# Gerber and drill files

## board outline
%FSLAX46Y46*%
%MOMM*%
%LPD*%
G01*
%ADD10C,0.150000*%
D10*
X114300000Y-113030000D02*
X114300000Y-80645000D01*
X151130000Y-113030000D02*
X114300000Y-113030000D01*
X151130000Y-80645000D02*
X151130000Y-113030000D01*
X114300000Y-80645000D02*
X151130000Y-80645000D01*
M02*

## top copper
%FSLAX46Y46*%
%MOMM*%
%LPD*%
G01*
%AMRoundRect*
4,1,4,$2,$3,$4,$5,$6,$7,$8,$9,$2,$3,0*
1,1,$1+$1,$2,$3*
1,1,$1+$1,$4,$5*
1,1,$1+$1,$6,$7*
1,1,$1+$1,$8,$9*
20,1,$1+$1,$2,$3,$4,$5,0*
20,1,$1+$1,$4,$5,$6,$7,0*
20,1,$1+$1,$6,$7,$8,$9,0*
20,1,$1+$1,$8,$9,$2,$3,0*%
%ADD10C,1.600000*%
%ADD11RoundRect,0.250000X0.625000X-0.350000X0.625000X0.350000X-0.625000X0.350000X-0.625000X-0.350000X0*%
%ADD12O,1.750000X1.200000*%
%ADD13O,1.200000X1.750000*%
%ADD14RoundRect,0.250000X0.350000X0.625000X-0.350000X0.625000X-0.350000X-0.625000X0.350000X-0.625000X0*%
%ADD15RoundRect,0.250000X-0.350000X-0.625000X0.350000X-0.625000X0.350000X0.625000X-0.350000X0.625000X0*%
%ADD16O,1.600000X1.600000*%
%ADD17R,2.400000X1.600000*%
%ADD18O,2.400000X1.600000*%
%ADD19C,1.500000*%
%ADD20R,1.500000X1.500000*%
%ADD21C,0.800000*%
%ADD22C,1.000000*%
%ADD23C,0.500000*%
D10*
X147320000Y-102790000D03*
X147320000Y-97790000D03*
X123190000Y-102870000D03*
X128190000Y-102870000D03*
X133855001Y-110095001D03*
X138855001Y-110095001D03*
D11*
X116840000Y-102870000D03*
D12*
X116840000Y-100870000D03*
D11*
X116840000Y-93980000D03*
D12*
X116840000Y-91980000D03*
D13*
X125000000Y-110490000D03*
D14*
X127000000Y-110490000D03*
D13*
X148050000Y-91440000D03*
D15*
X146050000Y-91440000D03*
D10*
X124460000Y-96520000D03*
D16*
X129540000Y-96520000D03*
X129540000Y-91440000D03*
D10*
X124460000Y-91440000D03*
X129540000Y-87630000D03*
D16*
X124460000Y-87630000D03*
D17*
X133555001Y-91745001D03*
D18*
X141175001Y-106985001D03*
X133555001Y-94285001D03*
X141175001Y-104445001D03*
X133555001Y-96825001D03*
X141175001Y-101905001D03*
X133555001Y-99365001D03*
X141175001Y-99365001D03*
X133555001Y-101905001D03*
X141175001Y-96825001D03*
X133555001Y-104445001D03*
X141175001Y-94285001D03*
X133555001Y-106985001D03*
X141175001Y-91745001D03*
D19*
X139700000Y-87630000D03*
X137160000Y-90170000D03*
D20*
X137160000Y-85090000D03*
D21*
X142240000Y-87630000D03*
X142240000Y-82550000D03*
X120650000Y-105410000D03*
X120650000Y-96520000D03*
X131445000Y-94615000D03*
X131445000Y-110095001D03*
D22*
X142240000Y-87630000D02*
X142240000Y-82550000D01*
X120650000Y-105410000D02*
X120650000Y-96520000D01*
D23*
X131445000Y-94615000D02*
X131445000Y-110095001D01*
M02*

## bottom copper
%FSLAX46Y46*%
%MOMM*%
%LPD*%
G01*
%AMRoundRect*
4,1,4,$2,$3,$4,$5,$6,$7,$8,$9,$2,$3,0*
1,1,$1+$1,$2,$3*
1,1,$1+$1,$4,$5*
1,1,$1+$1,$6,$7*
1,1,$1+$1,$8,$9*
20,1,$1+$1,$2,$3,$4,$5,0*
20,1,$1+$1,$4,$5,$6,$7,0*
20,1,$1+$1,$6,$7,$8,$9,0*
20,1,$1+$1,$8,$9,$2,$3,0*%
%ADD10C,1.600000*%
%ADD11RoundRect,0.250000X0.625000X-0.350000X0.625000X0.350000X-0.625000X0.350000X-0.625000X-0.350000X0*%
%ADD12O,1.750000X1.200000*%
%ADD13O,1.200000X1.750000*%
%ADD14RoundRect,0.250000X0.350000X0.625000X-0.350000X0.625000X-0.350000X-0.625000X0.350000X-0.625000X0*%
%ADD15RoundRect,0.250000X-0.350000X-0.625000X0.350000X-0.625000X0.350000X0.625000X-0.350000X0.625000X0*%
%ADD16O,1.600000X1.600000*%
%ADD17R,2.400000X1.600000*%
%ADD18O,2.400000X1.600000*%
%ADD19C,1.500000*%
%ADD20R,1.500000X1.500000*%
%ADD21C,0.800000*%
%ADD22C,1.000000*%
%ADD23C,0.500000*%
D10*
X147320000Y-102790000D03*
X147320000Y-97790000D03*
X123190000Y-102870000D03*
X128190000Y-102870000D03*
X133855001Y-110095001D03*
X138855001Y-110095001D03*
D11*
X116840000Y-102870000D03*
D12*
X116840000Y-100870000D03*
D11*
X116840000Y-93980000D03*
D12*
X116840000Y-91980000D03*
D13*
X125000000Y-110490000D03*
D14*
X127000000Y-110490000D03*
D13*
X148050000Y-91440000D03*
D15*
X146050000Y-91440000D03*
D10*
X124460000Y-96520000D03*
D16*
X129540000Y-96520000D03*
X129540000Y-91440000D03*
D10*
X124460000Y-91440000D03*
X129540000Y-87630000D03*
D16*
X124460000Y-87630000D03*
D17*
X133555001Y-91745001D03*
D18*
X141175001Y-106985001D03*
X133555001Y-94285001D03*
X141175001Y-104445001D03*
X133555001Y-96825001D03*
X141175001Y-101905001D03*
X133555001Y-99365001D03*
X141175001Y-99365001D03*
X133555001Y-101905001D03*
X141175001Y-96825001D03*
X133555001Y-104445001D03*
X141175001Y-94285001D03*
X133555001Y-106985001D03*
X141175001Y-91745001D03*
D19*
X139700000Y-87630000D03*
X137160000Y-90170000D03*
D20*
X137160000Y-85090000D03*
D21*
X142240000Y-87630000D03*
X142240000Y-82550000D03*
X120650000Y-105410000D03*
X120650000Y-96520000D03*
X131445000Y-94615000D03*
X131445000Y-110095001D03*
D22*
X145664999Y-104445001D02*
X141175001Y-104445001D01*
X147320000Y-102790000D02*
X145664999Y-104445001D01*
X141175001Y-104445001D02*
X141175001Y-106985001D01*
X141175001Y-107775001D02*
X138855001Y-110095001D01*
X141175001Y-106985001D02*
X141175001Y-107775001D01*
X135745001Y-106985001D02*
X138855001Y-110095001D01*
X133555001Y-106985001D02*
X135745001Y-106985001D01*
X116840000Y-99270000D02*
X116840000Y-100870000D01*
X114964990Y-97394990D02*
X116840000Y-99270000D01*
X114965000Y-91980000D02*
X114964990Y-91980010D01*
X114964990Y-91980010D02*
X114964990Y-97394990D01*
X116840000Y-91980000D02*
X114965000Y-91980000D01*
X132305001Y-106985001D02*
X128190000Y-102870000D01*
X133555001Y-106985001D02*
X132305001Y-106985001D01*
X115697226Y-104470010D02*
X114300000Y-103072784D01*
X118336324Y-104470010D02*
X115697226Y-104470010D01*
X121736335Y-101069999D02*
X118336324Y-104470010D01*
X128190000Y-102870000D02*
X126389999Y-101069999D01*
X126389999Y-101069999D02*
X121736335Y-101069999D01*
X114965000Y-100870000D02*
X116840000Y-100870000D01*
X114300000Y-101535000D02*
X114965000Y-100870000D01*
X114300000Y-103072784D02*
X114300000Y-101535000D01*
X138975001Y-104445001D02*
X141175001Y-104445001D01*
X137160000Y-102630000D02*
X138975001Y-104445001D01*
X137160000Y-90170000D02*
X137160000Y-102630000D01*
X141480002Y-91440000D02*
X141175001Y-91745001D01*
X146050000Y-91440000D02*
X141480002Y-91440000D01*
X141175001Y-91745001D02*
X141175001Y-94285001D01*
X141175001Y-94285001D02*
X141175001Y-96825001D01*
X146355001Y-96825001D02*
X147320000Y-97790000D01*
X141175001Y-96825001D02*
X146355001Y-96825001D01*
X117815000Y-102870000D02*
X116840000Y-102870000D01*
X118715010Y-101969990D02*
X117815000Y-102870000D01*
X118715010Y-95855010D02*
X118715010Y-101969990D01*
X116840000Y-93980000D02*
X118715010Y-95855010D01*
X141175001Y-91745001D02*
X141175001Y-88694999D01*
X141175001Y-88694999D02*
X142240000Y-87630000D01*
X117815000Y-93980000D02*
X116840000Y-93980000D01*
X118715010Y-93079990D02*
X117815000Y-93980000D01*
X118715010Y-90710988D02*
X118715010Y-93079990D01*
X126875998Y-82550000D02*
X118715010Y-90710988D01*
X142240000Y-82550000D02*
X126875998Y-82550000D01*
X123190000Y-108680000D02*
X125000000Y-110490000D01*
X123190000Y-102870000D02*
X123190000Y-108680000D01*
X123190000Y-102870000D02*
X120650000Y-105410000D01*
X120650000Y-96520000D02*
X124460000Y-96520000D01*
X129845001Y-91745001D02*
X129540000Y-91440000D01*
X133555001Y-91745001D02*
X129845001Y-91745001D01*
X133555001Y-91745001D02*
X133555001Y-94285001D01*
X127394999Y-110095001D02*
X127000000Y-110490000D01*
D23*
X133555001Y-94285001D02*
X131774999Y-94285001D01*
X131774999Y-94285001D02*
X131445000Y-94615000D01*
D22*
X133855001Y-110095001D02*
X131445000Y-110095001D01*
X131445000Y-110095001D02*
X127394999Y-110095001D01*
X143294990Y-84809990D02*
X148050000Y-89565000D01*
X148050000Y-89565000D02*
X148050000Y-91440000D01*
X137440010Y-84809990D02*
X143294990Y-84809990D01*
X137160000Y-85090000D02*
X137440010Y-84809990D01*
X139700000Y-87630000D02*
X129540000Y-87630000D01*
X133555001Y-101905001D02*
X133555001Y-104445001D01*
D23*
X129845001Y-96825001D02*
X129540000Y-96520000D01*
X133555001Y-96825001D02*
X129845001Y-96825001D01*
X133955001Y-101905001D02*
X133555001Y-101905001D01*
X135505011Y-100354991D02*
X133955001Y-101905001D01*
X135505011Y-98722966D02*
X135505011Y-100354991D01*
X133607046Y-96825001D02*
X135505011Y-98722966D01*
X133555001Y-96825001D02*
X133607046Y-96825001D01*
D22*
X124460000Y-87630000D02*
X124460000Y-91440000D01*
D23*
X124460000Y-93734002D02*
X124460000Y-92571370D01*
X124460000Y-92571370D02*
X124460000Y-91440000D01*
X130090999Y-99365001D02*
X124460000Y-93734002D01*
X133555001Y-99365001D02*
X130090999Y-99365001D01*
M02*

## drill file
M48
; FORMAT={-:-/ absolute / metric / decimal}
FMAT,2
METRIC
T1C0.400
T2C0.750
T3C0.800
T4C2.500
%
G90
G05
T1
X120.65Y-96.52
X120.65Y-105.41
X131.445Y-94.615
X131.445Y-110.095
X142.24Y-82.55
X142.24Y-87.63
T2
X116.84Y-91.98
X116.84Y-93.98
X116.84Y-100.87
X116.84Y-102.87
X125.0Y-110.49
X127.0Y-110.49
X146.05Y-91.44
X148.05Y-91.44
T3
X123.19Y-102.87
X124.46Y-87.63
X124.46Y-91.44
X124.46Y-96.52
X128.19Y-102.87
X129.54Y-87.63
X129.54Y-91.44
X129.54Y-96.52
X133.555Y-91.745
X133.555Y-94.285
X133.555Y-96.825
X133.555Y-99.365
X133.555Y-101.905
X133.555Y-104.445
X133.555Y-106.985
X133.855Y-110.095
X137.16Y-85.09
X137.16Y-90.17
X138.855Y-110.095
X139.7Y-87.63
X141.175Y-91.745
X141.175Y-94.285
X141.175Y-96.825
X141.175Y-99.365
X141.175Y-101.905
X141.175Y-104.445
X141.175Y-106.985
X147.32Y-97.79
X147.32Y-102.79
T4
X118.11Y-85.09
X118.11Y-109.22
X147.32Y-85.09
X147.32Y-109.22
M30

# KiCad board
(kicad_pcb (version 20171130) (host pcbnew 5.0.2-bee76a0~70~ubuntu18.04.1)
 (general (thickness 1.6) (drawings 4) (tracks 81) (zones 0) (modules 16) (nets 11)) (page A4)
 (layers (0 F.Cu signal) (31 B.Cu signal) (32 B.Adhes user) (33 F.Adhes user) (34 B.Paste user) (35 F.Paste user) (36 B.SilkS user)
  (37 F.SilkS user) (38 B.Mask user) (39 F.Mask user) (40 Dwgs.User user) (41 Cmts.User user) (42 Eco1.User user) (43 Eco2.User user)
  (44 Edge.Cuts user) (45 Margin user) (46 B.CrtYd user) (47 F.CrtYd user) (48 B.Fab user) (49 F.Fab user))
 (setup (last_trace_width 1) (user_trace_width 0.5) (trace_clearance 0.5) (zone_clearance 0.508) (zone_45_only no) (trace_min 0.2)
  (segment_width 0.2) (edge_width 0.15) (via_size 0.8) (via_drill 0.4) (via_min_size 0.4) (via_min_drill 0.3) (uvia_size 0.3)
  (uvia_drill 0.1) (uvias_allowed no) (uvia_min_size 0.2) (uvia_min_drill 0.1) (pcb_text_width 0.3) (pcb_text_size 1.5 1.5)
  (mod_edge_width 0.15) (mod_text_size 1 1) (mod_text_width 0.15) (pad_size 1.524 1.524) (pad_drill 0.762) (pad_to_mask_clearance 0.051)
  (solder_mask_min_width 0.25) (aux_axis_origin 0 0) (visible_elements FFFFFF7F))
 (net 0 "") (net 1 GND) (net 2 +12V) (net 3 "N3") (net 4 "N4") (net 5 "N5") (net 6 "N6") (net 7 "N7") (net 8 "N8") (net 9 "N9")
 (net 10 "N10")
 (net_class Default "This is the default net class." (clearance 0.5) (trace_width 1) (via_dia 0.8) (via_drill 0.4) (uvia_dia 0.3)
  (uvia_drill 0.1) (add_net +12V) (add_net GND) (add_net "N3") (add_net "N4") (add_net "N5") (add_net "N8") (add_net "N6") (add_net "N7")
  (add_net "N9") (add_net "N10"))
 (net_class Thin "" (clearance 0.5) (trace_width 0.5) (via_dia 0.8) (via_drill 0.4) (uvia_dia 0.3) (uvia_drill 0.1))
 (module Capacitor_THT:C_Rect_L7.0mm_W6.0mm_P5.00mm (layer F.Cu) (at 147.32 97.79 270)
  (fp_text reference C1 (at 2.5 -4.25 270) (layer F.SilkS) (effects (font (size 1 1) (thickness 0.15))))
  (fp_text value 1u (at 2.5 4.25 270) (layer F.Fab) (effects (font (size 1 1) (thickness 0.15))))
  (pad 2 thru_hole circle (at 5 0 270) (size 1.6 1.6) (drill 0.8) (layers *.Cu *.Mask) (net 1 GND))
  (pad 1 thru_hole circle (at 0 0 270) (size 1.6 1.6) (drill 0.8) (layers *.Cu *.Mask) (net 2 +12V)))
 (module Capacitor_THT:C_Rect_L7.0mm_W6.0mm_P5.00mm (layer F.Cu) (at 123.19 102.87)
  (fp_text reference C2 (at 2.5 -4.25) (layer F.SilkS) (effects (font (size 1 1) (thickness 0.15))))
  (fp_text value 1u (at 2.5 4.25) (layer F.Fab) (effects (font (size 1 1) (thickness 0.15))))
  (pad 1 thru_hole circle (at 0 0) (size 1.6 1.6) (drill 0.8) (layers *.Cu *.Mask) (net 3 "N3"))
  (pad 2 thru_hole circle (at 5 0) (size 1.6 1.6) (drill 0.8) (layers *.Cu *.Mask) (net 1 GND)))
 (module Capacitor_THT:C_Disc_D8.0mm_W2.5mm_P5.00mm (layer F.Cu) (at 133.855001 110.095001)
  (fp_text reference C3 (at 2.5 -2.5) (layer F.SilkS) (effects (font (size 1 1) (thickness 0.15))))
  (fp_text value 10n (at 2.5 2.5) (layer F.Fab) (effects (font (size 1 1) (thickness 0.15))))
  (pad 1 thru_hole circle (at 0 0) (size 1.6 1.6) (drill 0.8) (layers *.Cu *.Mask) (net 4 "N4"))
  (pad 2 thru_hole circle (at 5 0) (size 1.6 1.6) (drill 0.8) (layers *.Cu *.Mask) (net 1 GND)))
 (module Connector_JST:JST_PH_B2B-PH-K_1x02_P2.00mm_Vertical (layer F.Cu) (at 116.84 102.87 90)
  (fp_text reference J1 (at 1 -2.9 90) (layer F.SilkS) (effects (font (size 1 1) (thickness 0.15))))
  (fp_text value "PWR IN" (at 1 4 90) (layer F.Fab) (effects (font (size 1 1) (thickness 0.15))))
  (pad 1 thru_hole roundrect (at 0 0 90) (size 1.2 1.75) (drill 0.75) (layers *.Cu *.Mask) (roundrect_rratio 0.208333) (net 2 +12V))
  (pad 2 thru_hole oval (at 2 0 90) (size 1.2 1.75) (drill 0.75) (layers *.Cu *.Mask) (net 1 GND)))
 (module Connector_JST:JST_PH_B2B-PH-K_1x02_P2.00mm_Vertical (layer F.Cu) (at 116.84 93.98 90)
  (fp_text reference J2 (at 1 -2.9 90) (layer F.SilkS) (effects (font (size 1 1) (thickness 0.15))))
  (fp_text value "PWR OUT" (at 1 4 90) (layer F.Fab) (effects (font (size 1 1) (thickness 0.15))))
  (pad 1 thru_hole roundrect (at 0 0 90) (size 1.2 1.75) (drill 0.75) (layers *.Cu *.Mask) (roundrect_rratio 0.208333) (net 2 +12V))
  (pad 2 thru_hole oval (at 2 0 90) (size 1.2 1.75) (drill 0.75) (layers *.Cu *.Mask) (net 1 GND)))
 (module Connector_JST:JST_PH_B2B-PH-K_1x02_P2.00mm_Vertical (layer F.Cu) (at 127 110.49 180)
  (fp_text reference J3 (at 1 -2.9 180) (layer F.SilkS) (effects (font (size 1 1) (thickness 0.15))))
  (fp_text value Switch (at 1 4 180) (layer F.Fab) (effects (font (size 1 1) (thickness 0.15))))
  (pad 2 thru_hole oval (at 2 0 180) (size 1.2 1.75) (drill 0.75) (layers *.Cu *.Mask) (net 3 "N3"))
  (pad 1 thru_hole roundrect (at 0 0 180) (size 1.2 1.75) (drill 0.75) (layers *.Cu *.Mask) (roundrect_rratio 0.208333) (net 4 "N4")))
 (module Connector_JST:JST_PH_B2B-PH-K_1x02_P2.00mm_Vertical (layer F.Cu) (at 146.05 91.44)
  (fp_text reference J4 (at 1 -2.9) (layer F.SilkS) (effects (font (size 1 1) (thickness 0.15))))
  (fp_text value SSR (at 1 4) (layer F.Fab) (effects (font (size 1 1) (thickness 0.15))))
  (pad 2 thru_hole oval (at 2 0) (size 1.2 1.75) (drill 0.75) (layers *.Cu *.Mask) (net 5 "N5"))
  (pad 1 thru_hole roundrect (at 0 0) (size 1.2 1.75) (drill 0.75) (layers *.Cu *.Mask) (roundrect_rratio 0.208333) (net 2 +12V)))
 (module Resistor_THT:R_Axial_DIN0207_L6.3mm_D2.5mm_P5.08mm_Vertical (layer F.Cu) (at 124.46 96.52)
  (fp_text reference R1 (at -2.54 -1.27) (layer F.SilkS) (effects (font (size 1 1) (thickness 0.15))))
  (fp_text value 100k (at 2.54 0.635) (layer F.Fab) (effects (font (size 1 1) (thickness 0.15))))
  (pad 1 thru_hole circle (at 0 0) (size 1.6 1.6) (drill 0.8) (layers *.Cu *.Mask) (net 3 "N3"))
  (pad 2 thru_hole oval (at 5.08 0) (size 1.6 1.6) (drill 0.8) (layers *.Cu *.Mask) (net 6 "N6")))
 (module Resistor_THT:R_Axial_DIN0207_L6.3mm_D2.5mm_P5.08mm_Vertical (layer F.Cu) (at 124.46 91.44)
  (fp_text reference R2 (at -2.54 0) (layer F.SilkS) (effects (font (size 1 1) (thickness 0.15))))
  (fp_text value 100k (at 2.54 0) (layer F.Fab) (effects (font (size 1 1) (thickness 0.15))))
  (pad 2 thru_hole oval (at 5.08 0) (size 1.6 1.6) (drill 0.8) (layers *.Cu *.Mask) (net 4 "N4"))
  (pad 1 thru_hole circle (at 0 0) (size 1.6 1.6) (drill 0.8) (layers *.Cu *.Mask) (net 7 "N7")))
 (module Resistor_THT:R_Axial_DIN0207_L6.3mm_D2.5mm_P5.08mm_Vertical (layer F.Cu) (at 129.54 87.63 180)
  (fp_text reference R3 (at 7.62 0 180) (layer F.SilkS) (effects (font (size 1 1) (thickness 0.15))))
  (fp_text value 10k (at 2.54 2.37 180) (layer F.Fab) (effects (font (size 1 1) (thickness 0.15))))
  (pad 1 thru_hole circle (at 0 0 180) (size 1.6 1.6) (drill 0.8) (layers *.Cu *.Mask) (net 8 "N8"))
  (pad 2 thru_hole oval (at 5.08 0 180) (size 1.6 1.6) (drill 0.8) (layers *.Cu *.Mask) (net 7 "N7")))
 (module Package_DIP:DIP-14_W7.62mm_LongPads (layer F.Cu) (at 133.555001 91.745001)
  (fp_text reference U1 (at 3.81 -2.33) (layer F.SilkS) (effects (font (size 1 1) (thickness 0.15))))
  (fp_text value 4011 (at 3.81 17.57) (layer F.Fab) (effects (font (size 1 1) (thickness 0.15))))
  (pad 1 thru_hole rect (at 0 0) (size 2.4 1.6) (drill 0.8) (layers *.Cu *.Mask) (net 4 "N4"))
  (pad 8 thru_hole oval (at 7.62 15.24) (size 2.4 1.6) (drill 0.8) (layers *.Cu *.Mask) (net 1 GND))
  (pad 2 thru_hole oval (at 0 2.54) (size 2.4 1.6) (drill 0.8) (layers *.Cu *.Mask) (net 4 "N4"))
  (pad 9 thru_hole oval (at 7.62 12.7) (size 2.4 1.6) (drill 0.8) (layers *.Cu *.Mask) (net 1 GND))
  (pad 3 thru_hole oval (at 0 5.08) (size 2.4 1.6) (drill 0.8) (layers *.Cu *.Mask) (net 6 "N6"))
  (pad 10 thru_hole oval (at 7.62 10.16) (size 2.4 1.6) (drill 0.8) (layers *.Cu *.Mask) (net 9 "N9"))
  (pad 4 thru_hole oval (at 0 7.62) (size 2.4 1.6) (drill 0.8) (layers *.Cu *.Mask) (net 7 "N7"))
  (pad 11 thru_hole oval (at 7.62 7.62) (size 2.4 1.6) (drill 0.8) (layers *.Cu *.Mask) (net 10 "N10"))
  (pad 5 thru_hole oval (at 0 10.16) (size 2.4 1.6) (drill 0.8) (layers *.Cu *.Mask) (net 6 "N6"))
  (pad 12 thru_hole oval (at 7.62 5.08) (size 2.4 1.6) (drill 0.8) (layers *.Cu *.Mask) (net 2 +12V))
  (pad 6 thru_hole oval (at 0 12.7) (size 2.4 1.6) (drill 0.8) (layers *.Cu *.Mask) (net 6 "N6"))
  (pad 13 thru_hole oval (at 7.62 2.54) (size 2.4 1.6) (drill 0.8) (layers *.Cu *.Mask) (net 2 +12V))
  (pad 7 thru_hole oval (at 0 15.24) (size 2.4 1.6) (drill 0.8) (layers *.Cu *.Mask) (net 1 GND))
  (pad 14 thru_hole oval (at 7.62 0) (size 2.4 1.6) (drill 0.8) (layers *.Cu *.Mask) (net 2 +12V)))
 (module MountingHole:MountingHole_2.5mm (layer F.Cu) (at 118.11 85.09)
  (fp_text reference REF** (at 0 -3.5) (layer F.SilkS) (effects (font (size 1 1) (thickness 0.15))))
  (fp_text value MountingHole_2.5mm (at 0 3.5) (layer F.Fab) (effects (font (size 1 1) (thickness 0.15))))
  (pad 1 np_thru_hole circle (at 0 0) (size 2.5 2.5) (drill 2.5) (layers *.Cu *.Mask)))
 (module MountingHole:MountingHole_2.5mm (layer F.Cu) (at 147.32 85.09)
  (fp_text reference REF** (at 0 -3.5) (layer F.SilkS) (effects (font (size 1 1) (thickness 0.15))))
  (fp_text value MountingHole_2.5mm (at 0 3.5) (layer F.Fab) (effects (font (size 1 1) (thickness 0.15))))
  (pad 1 np_thru_hole circle (at 0 0) (size 2.5 2.5) (drill 2.5) (layers *.Cu *.Mask)))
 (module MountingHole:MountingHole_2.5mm (layer F.Cu) (at 118.11 109.22)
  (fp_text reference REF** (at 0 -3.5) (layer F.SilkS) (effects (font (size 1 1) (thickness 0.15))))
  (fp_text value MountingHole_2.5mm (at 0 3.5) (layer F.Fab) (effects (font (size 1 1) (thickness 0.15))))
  (pad 1 np_thru_hole circle (at 0 0) (size 2.5 2.5) (drill 2.5) (layers *.Cu *.Mask)))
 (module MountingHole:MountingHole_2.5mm (layer F.Cu) (at 147.32 109.22)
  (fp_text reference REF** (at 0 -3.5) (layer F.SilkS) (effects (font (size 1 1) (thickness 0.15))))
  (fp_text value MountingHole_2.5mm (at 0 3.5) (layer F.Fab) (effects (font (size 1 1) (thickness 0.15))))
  (pad 1 np_thru_hole circle (at 0 0) (size 2.5 2.5) (drill 2.5) (layers *.Cu *.Mask)))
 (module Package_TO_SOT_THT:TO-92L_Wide (layer F.Cu) (at 137.16 85.09 270)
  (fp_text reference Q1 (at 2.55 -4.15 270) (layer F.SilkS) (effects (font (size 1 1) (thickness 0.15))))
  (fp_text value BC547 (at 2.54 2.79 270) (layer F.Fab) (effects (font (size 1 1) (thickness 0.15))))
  (pad 2 thru_hole circle (at 2.54 -2.54) (size 1.5 1.5) (drill 0.8) (layers *.Cu *.Mask) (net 8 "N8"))
  (pad 3 thru_hole circle (at 5.08 0) (size 1.5 1.5) (drill 0.8) (layers *.Cu *.Mask) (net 1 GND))
  (pad 1 thru_hole rect (at 0 0) (size 1.5 1.5) (drill 0.8) (layers *.Cu *.Mask) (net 5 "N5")))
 (gr_line (start 114.3 113.03) (end 114.3 80.645) (layer Edge.Cuts) (width 0.15))
 (gr_line (start 151.13 113.03) (end 114.3 113.03) (layer Edge.Cuts) (width 0.15))
 (gr_line (start 151.13 80.645) (end 151.13 113.03) (layer Edge.Cuts) (width 0.15))
 (gr_line (start 114.3 80.645) (end 151.13 80.645) (layer Edge.Cuts) (width 0.15))
 (segment (start 145.664999 104.445001) (end 141.175001 104.445001) (width 1) (layer B.Cu) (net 1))
 (segment (start 147.32 102.79) (end 145.664999 104.445001) (width 1) (layer B.Cu) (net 1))
 (segment (start 141.175001 104.445001) (end 141.175001 106.985001) (width 1) (layer B.Cu) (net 1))
 (segment (start 141.175001 107.775001) (end 138.855001 110.095001) (width 1) (layer B.Cu) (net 1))
 (segment (start 141.175001 106.985001) (end 141.175001 107.775001) (width 1) (layer B.Cu) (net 1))
 (segment (start 135.745001 106.985001) (end 138.855001 110.095001) (width 1) (layer B.Cu) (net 1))
 (segment (start 133.555001 106.985001) (end 135.745001 106.985001) (width 1) (layer B.Cu) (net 1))
 (segment (start 116.84 99.27) (end 116.84 100.87) (width 1) (layer B.Cu) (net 1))
 (segment (start 114.96499 97.39499) (end 116.84 99.27) (width 1) (layer B.Cu) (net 1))
 (segment (start 114.965 91.98) (end 114.96499 91.98001) (width 1) (layer B.Cu) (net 1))
 (segment (start 114.96499 91.98001) (end 114.96499 97.39499) (width 1) (layer B.Cu) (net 1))
 (segment (start 116.84 91.98) (end 114.965 91.98) (width 1) (layer B.Cu) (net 1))
 (segment (start 132.305001 106.985001) (end 128.19 102.87) (width 1) (layer B.Cu) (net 1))
 (segment (start 133.555001 106.985001) (end 132.305001 106.985001) (width 1) (layer B.Cu) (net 1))
 (segment (start 115.697226 104.47001) (end 114.3 103.072784) (width 1) (layer B.Cu) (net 1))
 (segment (start 118.336324 104.47001) (end 115.697226 104.47001) (width 1) (layer B.Cu) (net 1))
 (segment (start 121.736335 101.069999) (end 118.336324 104.47001) (width 1) (layer B.Cu) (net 1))
 (segment (start 128.19 102.87) (end 126.389999 101.069999) (width 1) (layer B.Cu) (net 1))
 (segment (start 126.389999 101.069999) (end 121.736335 101.069999) (width 1) (layer B.Cu) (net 1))
 (segment (start 114.965 100.87) (end 116.84 100.87) (width 1) (layer B.Cu) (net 1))
 (segment (start 114.3 101.535) (end 114.965 100.87) (width 1) (layer B.Cu) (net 1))
 (segment (start 114.3 103.072784) (end 114.3 101.535) (width 1) (layer B.Cu) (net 1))
 (segment (start 138.975001 104.445001) (end 141.175001 104.445001) (width 1) (layer B.Cu) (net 1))
 (segment (start 137.16 102.63) (end 138.975001 104.445001) (width 1) (layer B.Cu) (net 1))
 (segment (start 137.16 90.17) (end 137.16 102.63) (width 1) (layer B.Cu) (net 1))
 (segment (start 141.480002 91.44) (end 141.175001 91.745001) (width 1) (layer B.Cu) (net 2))
 (segment (start 146.05 91.44) (end 141.480002 91.44) (width 1) (layer B.Cu) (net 2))
 (segment (start 141.175001 91.745001) (end 141.175001 94.285001) (width 1) (layer B.Cu) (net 2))
 (segment (start 141.175001 94.285001) (end 141.175001 96.825001) (width 1) (layer B.Cu) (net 2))
 (segment (start 146.355001 96.825001) (end 147.32 97.79) (width 1) (layer B.Cu) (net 2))
 (segment (start 141.175001 96.825001) (end 146.355001 96.825001) (width 1) (layer B.Cu) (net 2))
 (segment (start 117.815 102.87) (end 116.84 102.87) (width 1) (layer B.Cu) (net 2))
 (segment (start 118.71501 101.96999) (end 117.815 102.87) (width 1) (layer B.Cu) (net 2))
 (segment (start 118.71501 95.85501) (end 118.71501 101.96999) (width 1) (layer B.Cu) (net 2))
 (segment (start 116.84 93.98) (end 118.71501 95.85501) (width 1) (layer B.Cu) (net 2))
 (via (at 142.24 87.63) (size 0.8) (drill 0.4) (layers F.Cu B.Cu) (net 2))
 (segment (start 141.175001 91.745001) (end 141.175001 88.694999) (width 1) (layer B.Cu) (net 2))
 (segment (start 141.175001 88.694999) (end 142.24 87.63) (width 1) (layer B.Cu) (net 2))
 (via (at 142.24 82.55) (size 0.8) (drill 0.4) (layers F.Cu B.Cu) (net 2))
 (segment (start 142.24 87.63) (end 142.24 82.55) (width 1) (layer F.Cu) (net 2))
 (segment (start 117.815 93.98) (end 116.84 93.98) (width 1) (layer B.Cu) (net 2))
 (segment (start 118.71501 93.07999) (end 117.815 93.98) (width 1) (layer B.Cu) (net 2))
 (segment (start 118.71501 90.710988) (end 118.71501 93.07999) (width 1) (layer B.Cu) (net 2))
 (segment (start 126.875998 82.55) (end 118.71501 90.710988) (width 1) (layer B.Cu) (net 2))
 (segment (start 142.24 82.55) (end 126.875998 82.55) (width 1) (layer B.Cu) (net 2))
 (segment (start 123.19 108.68) (end 125 110.49) (width 1) (layer B.Cu) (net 3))
 (segment (start 123.19 102.87) (end 123.19 108.68) (width 1) (layer B.Cu) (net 3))
 (via (at 120.65 105.41) (size 0.8) (drill 0.4) (layers F.Cu B.Cu) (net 3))
 (segment (start 123.19 102.87) (end 120.65 105.41) (width 1) (layer B.Cu) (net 3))
 (via (at 120.65 96.52) (size 0.8) (drill 0.4) (layers F.Cu B.Cu) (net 3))
 (segment (start 120.65 105.41) (end 120.65 96.52) (width 1) (layer F.Cu) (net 3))
 (segment (start 120.65 96.52) (end 124.46 96.52) (width 1) (layer B.Cu) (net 3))
 (segment (start 129.845001 91.745001) (end 129.54 91.44) (width 1) (layer B.Cu) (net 4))
 (segment (start 133.555001 91.745001) (end 129.845001 91.745001) (width 1) (layer B.Cu) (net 4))
 (segment (start 133.555001 91.745001) (end 133.555001 94.285001) (width 1) (layer B.Cu) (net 4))
 (segment (start 127.394999 110.095001) (end 127 110.49) (width 1) (layer B.Cu) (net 4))
 (via (at 131.445 94.615) (size 0.8) (drill 0.4) (layers F.Cu B.Cu) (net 4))
 (segment (start 133.555001 94.285001) (end 131.774999 94.285001) (width 0.5) (layer B.Cu) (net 4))
 (segment (start 131.774999 94.285001) (end 131.445 94.615) (width 0.5) (layer B.Cu) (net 4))
 (via (at 131.445 110.095001) (size 0.8) (drill 0.4) (layers F.Cu B.Cu) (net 4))
 (segment (start 131.445 94.615) (end 131.445 110.095001) (width 0.5) (layer F.Cu) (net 4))
 (segment (start 133.855001 110.095001) (end 131.445 110.095001) (width 1) (layer B.Cu) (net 4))
 (segment (start 131.445 110.095001) (end 127.394999 110.095001) (width 1) (layer B.Cu) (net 4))
 (segment (start 143.29499 84.80999) (end 148.05 89.565) (width 1) (layer B.Cu) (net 5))
 (segment (start 148.05 89.565) (end 148.05 91.44) (width 1) (layer B.Cu) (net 5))
 (segment (start 137.44001 84.80999) (end 143.29499 84.80999) (width 1) (layer B.Cu) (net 5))
 (segment (start 137.16 85.09) (end 137.44001 84.80999) (width 1) (layer B.Cu) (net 5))
 (segment (start 139.7 87.63) (end 129.54 87.63) (width 1) (layer B.Cu) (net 8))
 (segment (start 133.555001 101.905001) (end 133.555001 104.445001) (width 1) (layer B.Cu) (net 6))
 (segment (start 129.845001 96.825001) (end 129.54 96.52) (width 0.5) (layer B.Cu) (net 6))
 (segment (start 133.555001 96.825001) (end 129.845001 96.825001) (width 0.5) (layer B.Cu) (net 6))
 (segment (start 133.955001 101.905001) (end 133.555001 101.905001) (width 0.5) (layer B.Cu) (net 6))
 (segment (start 135.505011 100.354991) (end 133.955001 101.905001) (width 0.5) (layer B.Cu) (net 6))
 (segment (start 135.505011 98.722966) (end 135.505011 100.354991) (width 0.5) (layer B.Cu) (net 6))
 (segment (start 133.607046 96.825001) (end 135.505011 98.722966) (width 0.5) (layer B.Cu) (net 6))
 (segment (start 133.555001 96.825001) (end 133.607046 96.825001) (width 0.5) (layer B.Cu) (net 6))
 (segment (start 124.46 87.63) (end 124.46 91.44) (width 1) (layer B.Cu) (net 7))
 (segment (start 124.46 93.734002) (end 124.46 92.57137) (width 0.5) (layer B.Cu) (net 7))
 (segment (start 124.46 92.57137) (end 124.46 91.44) (width 0.5) (layer B.Cu) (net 7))
 (segment (start 130.090999 99.365001) (end 124.46 93.734002) (width 0.5) (layer B.Cu) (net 7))
 (segment (start 133.555001 99.365001) (end 130.090999 99.365001) (width 0.5) (layer B.Cu) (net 7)))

